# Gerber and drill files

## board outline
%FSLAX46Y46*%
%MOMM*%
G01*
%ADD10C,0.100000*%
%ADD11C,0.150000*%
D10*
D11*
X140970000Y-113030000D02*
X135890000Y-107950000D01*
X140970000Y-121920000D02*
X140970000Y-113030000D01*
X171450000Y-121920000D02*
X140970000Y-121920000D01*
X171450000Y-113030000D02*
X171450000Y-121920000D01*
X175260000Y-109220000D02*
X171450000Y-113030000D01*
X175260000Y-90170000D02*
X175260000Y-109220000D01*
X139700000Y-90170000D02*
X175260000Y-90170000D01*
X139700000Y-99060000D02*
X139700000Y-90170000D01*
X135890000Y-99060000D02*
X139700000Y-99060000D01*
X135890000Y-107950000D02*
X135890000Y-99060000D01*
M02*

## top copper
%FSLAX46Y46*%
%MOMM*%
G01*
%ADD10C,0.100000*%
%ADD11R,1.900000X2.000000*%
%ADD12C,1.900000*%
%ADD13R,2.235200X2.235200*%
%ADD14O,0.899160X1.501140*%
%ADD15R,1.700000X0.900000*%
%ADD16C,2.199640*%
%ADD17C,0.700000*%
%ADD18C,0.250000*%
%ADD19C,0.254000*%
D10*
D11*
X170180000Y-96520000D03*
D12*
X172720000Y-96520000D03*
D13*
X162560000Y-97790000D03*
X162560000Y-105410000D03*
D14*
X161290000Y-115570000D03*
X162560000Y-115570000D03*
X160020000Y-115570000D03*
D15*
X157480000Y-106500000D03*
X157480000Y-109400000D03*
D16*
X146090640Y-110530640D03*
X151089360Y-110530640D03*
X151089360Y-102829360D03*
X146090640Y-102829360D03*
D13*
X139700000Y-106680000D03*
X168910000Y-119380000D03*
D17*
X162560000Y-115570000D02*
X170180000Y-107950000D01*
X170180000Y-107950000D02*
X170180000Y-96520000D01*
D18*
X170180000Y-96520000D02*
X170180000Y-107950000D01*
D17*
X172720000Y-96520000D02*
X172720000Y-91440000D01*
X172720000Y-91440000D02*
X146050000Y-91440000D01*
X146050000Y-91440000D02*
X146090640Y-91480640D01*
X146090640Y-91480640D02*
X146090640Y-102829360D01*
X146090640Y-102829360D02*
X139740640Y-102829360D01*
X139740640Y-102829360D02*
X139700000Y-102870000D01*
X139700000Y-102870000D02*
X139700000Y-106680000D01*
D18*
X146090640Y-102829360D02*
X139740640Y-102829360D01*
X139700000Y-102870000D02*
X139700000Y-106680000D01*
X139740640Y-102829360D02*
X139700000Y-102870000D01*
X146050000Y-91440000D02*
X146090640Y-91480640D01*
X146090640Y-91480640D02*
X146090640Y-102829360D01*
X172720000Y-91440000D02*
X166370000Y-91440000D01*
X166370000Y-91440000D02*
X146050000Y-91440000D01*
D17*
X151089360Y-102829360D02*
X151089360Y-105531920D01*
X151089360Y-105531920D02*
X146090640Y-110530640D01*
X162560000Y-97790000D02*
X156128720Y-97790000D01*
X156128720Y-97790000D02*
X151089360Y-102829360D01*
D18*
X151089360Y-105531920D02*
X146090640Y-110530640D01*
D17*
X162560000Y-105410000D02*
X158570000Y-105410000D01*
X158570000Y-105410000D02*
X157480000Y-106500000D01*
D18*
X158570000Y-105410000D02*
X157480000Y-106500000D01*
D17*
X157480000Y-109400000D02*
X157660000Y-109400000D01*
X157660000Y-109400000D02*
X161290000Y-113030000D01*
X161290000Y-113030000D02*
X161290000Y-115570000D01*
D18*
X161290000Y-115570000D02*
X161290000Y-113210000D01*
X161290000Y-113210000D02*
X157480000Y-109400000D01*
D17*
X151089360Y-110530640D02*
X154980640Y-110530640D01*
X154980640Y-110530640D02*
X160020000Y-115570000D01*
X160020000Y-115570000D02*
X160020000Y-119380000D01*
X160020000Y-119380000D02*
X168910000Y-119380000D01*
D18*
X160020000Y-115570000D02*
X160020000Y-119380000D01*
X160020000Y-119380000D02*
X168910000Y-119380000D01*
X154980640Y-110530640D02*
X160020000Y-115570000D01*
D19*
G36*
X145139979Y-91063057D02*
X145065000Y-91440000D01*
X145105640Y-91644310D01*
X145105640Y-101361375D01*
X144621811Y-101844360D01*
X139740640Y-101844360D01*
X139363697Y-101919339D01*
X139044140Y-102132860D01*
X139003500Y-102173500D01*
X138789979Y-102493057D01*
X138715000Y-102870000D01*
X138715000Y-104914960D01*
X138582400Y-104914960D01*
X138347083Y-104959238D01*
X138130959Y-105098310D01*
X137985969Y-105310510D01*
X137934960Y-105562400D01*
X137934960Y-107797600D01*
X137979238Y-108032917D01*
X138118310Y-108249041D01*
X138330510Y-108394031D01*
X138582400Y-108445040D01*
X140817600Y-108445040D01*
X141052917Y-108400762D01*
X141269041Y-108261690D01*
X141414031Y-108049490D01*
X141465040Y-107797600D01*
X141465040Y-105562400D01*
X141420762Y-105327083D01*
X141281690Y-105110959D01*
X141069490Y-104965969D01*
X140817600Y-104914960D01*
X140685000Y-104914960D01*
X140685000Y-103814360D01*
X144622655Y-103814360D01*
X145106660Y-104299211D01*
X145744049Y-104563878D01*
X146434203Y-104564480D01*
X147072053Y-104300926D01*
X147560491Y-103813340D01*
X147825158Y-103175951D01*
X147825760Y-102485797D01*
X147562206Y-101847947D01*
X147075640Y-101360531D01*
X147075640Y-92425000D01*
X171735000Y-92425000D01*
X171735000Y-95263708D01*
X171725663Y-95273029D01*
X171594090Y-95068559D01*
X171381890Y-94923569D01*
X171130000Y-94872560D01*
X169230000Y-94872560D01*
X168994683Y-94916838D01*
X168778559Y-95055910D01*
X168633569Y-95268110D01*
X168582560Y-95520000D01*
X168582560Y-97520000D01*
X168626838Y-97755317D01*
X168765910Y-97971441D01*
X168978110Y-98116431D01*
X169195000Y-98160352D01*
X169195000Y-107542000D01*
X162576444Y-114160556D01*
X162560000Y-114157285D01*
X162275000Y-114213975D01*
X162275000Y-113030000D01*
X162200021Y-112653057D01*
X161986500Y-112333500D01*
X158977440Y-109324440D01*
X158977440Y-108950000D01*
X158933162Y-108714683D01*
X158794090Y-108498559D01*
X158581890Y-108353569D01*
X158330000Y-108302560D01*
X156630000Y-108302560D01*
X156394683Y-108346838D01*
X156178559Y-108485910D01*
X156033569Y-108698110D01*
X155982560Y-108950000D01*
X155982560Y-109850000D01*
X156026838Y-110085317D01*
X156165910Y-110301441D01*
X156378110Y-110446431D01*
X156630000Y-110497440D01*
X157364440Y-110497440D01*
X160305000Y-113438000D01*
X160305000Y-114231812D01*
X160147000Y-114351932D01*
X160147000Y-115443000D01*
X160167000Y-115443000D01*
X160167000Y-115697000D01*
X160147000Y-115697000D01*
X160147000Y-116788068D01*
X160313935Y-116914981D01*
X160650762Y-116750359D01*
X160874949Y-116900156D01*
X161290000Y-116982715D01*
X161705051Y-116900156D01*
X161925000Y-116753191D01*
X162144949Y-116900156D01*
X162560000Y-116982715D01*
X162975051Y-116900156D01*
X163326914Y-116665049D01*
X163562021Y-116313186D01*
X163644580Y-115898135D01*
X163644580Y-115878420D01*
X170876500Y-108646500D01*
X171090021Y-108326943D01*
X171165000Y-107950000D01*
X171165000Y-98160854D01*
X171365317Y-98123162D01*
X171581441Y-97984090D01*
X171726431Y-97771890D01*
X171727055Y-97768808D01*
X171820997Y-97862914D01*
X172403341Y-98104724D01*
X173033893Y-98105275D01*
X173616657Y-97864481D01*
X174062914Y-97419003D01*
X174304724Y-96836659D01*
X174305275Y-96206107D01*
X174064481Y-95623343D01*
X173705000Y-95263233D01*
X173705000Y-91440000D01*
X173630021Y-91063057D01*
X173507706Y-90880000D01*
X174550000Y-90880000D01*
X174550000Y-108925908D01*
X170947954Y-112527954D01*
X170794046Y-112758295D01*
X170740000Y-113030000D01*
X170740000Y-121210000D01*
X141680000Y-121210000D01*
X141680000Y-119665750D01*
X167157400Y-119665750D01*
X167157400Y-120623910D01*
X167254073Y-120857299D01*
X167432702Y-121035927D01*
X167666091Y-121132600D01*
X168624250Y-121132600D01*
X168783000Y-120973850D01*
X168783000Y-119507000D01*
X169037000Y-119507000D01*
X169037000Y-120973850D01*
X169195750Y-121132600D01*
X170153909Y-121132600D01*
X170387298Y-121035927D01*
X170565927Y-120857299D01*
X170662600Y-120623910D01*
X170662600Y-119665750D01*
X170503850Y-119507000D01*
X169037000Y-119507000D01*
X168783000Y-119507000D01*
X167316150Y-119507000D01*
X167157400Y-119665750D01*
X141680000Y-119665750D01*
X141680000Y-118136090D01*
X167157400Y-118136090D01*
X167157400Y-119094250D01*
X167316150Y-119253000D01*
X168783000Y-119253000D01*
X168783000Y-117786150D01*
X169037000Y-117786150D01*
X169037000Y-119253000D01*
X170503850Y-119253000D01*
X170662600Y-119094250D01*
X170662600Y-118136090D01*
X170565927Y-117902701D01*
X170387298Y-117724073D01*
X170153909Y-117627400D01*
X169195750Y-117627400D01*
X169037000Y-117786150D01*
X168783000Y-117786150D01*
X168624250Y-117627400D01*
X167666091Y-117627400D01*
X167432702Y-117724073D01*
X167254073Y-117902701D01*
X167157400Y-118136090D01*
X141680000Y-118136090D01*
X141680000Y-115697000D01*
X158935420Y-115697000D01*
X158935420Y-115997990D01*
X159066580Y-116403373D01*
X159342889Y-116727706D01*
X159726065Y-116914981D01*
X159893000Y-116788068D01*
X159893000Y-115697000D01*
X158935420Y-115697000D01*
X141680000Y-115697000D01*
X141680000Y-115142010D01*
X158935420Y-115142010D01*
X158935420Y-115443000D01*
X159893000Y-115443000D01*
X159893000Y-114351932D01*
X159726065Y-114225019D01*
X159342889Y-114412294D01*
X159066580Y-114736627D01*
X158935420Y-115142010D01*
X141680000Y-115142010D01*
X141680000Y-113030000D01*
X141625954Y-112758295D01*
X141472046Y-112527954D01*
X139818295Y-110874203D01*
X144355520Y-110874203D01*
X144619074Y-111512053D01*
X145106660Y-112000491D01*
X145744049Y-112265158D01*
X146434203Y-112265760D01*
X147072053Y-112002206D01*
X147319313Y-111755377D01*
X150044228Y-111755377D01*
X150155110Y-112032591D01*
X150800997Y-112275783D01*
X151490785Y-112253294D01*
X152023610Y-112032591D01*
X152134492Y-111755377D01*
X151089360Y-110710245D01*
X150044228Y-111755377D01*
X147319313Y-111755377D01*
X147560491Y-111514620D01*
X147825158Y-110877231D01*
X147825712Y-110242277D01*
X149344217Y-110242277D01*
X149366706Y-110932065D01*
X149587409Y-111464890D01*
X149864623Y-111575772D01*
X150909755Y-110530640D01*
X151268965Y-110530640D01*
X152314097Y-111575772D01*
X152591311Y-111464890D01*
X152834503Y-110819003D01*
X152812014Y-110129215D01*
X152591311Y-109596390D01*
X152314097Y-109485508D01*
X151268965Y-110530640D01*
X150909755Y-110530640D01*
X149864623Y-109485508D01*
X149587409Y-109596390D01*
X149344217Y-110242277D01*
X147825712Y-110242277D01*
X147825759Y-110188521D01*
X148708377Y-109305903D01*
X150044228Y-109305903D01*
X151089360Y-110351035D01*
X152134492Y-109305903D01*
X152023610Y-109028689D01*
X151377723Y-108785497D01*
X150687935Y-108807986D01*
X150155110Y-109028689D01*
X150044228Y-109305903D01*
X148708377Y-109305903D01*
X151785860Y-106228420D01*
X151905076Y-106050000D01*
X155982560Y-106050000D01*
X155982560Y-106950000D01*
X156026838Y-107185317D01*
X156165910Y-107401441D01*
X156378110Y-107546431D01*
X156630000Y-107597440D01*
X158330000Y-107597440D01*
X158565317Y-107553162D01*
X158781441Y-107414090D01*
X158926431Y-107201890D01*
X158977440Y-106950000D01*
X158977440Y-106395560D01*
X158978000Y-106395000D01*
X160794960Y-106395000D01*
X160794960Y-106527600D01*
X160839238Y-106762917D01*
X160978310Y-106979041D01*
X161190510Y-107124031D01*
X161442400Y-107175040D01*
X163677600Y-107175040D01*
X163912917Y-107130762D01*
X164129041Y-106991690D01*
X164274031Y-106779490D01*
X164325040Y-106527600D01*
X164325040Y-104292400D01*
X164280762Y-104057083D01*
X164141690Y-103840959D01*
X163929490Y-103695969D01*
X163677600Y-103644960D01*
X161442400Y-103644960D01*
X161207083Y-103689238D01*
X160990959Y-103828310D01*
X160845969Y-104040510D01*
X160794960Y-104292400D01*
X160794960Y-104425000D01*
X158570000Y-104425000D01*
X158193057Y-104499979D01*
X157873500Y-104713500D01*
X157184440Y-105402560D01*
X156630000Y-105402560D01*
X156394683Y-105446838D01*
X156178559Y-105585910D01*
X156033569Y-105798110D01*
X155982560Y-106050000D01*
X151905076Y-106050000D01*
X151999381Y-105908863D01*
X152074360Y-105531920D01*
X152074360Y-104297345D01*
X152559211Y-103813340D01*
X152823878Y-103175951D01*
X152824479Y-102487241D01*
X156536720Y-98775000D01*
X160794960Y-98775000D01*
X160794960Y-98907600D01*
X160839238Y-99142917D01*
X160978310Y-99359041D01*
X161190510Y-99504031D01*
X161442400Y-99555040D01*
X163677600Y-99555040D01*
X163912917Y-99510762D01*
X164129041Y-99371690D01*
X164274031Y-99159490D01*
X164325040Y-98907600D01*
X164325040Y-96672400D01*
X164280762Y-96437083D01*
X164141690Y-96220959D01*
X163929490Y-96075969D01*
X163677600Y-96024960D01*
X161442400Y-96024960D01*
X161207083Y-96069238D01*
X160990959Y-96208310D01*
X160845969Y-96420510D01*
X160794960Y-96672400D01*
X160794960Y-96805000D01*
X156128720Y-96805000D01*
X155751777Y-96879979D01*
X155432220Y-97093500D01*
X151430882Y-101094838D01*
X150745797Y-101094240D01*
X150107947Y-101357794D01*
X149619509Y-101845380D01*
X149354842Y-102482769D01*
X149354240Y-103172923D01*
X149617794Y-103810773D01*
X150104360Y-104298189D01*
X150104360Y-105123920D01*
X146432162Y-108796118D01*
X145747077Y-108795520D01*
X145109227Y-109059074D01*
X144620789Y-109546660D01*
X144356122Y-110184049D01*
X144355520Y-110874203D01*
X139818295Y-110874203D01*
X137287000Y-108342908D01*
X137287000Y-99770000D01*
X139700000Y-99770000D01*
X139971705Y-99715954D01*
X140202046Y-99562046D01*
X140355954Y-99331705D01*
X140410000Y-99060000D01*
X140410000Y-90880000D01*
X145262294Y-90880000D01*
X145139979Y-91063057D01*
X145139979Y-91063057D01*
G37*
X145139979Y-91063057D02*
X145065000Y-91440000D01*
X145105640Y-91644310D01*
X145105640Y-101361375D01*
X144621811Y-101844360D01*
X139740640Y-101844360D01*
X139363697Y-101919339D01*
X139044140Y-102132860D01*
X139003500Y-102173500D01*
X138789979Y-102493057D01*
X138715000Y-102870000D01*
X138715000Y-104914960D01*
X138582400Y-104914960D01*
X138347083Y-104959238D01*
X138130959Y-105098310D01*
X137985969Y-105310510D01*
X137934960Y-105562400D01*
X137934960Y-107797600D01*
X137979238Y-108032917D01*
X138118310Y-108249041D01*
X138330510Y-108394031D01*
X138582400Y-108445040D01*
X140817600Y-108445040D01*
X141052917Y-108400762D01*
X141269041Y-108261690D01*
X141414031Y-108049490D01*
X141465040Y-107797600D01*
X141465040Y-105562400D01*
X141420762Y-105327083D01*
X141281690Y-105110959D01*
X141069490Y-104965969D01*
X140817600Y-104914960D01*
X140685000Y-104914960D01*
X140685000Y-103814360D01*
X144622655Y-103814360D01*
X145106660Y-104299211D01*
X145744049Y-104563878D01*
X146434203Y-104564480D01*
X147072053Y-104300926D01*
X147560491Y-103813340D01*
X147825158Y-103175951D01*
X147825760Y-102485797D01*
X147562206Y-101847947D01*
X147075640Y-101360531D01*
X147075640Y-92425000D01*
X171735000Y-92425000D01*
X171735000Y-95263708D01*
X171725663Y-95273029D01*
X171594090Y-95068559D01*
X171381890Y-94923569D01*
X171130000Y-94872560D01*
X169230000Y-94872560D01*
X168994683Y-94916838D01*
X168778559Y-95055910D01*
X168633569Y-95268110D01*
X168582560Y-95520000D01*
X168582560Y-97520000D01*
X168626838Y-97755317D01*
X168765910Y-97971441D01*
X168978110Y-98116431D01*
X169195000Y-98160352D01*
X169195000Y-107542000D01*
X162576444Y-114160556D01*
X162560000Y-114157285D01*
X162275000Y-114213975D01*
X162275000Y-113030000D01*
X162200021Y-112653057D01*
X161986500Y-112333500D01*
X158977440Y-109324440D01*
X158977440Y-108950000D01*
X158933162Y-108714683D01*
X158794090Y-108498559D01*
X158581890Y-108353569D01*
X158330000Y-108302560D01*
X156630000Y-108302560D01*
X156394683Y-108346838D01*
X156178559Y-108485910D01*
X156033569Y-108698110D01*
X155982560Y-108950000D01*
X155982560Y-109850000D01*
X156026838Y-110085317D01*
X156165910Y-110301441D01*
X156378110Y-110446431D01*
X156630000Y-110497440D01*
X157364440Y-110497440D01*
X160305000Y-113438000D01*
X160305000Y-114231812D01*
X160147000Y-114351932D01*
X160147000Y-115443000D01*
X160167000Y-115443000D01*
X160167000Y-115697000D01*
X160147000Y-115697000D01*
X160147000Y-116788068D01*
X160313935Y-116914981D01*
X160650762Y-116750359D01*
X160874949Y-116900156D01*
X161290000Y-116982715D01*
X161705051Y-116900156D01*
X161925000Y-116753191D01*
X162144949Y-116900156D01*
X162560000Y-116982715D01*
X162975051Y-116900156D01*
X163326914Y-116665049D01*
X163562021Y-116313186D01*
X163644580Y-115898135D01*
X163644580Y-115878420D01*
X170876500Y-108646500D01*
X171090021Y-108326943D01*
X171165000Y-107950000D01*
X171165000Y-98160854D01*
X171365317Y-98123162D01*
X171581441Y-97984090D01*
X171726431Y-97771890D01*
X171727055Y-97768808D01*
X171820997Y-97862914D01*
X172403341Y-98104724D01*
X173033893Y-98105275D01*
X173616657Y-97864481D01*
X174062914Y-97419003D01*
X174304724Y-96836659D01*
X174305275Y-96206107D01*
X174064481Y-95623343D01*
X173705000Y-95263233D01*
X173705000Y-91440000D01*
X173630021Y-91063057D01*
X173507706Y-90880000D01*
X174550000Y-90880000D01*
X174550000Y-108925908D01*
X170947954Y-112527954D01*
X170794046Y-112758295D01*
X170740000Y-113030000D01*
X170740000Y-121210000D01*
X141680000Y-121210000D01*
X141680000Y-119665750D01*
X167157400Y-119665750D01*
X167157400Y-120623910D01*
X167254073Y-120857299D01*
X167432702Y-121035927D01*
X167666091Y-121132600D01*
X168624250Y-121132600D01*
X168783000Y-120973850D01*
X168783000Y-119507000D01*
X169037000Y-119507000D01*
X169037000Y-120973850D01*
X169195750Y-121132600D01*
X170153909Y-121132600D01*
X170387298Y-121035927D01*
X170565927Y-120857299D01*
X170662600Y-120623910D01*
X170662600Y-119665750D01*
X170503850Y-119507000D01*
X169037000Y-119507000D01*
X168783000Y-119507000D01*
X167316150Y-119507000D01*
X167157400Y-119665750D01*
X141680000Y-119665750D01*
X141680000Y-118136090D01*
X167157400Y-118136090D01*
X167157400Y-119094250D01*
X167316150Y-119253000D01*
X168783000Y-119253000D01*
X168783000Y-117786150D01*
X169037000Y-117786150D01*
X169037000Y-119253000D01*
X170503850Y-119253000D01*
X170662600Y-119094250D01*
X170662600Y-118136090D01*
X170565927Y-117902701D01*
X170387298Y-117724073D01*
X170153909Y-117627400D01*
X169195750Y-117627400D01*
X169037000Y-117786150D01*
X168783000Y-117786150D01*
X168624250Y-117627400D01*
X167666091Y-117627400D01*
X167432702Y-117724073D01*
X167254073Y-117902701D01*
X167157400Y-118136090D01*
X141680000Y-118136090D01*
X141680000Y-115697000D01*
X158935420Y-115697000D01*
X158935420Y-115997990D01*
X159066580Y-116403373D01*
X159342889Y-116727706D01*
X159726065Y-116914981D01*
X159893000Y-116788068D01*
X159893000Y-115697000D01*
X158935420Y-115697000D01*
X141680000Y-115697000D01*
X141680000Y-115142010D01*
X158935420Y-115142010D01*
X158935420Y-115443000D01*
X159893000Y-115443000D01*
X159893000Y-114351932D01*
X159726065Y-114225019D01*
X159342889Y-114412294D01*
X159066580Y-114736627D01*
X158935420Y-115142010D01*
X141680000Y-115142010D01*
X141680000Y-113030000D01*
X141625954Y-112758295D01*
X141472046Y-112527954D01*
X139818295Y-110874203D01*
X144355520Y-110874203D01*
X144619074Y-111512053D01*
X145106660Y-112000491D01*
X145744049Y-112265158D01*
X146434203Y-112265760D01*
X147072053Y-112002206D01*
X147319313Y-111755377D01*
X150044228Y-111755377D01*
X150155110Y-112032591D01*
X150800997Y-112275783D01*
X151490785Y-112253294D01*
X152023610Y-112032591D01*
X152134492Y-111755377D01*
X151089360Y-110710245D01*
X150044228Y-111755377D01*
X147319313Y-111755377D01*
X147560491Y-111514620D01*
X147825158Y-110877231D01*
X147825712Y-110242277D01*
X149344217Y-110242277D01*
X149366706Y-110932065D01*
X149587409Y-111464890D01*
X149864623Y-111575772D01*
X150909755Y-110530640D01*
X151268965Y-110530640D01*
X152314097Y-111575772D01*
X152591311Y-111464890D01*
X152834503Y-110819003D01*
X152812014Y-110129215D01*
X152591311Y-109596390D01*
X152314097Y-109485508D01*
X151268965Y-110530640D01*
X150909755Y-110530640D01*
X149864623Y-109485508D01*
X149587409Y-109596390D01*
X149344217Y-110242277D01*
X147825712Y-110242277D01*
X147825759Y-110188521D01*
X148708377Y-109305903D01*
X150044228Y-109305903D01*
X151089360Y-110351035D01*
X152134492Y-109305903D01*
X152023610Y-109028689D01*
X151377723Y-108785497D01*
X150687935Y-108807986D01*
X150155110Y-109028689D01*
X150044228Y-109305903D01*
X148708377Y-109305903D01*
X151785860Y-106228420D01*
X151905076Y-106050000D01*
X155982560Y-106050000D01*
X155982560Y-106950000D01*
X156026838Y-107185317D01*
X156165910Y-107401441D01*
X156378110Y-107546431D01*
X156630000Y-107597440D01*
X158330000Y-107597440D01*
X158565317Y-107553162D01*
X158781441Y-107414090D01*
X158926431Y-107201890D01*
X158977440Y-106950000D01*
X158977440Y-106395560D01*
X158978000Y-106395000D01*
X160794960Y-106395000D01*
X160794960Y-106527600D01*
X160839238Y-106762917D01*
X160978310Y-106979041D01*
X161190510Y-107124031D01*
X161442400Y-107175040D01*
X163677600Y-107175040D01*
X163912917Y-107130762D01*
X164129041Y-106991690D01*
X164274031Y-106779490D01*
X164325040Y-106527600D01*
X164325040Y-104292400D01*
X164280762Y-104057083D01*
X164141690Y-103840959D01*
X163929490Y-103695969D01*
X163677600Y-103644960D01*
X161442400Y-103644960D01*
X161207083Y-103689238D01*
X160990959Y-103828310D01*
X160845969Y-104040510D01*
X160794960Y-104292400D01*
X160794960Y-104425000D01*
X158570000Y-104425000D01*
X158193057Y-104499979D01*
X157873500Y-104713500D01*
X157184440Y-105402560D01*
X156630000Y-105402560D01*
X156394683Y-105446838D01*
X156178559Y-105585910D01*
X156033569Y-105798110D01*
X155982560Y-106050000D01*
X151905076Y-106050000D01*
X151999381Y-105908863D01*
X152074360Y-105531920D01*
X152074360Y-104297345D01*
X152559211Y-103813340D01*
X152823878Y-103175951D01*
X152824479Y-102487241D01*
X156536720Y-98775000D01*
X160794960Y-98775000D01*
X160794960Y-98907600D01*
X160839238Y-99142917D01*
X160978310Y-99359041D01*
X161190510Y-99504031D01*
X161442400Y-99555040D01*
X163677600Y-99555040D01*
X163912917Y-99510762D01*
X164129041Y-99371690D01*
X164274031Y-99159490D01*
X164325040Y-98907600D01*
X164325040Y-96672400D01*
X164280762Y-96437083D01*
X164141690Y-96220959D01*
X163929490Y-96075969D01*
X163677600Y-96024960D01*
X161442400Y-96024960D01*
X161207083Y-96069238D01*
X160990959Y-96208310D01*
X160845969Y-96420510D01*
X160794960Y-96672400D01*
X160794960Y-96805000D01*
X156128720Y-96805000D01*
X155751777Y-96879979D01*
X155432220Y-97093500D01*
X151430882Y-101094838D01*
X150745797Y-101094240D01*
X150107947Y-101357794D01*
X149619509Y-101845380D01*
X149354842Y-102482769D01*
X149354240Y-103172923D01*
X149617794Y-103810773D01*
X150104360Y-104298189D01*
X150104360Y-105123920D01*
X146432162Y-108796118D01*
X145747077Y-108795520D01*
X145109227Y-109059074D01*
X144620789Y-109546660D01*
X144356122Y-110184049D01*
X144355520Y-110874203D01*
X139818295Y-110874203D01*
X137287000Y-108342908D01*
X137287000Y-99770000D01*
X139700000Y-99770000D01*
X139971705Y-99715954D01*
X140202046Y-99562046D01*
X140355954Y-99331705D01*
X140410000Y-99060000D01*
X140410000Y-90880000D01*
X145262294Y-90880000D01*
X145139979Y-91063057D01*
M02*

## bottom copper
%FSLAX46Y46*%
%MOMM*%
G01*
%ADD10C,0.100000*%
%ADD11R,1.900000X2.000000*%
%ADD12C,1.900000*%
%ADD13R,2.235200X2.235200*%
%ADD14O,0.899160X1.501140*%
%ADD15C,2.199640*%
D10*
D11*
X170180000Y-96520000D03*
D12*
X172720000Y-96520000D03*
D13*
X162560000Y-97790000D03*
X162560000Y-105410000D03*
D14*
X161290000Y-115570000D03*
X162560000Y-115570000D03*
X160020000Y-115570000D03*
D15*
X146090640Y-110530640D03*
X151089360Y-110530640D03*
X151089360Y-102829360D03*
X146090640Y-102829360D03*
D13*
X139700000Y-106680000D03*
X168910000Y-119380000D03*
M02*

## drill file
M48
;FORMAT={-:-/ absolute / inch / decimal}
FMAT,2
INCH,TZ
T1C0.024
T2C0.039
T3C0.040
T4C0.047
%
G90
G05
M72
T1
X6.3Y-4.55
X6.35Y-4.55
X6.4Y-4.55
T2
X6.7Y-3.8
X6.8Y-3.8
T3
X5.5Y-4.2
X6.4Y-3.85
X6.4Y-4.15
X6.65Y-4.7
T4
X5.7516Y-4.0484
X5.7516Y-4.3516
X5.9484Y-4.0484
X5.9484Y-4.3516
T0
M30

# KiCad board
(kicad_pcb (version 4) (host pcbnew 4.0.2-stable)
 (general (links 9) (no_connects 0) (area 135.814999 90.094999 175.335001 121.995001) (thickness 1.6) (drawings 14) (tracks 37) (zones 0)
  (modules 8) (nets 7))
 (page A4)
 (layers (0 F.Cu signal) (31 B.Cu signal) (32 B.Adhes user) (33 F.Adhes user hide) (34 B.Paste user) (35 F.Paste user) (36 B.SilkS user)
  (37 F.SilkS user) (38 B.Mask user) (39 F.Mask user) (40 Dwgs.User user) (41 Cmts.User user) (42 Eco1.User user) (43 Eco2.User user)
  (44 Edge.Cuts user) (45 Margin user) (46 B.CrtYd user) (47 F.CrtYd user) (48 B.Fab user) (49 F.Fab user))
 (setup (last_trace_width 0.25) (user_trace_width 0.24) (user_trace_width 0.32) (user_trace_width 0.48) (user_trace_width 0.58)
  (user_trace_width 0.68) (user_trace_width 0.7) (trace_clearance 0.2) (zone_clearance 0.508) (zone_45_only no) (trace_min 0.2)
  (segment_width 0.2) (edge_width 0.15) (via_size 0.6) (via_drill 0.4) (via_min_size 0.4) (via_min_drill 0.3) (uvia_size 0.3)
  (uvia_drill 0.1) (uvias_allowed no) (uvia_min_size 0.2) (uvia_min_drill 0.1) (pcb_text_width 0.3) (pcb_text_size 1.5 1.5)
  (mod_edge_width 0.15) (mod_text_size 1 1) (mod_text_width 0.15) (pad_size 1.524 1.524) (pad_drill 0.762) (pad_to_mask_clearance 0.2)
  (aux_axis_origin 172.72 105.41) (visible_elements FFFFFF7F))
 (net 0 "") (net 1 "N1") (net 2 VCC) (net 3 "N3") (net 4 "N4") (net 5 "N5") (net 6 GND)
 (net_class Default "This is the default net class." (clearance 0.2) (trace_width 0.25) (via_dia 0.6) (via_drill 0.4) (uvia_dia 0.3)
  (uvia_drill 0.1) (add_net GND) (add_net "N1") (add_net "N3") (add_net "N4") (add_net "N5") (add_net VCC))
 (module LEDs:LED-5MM (layer F.Cu) (at 170.18 96.52)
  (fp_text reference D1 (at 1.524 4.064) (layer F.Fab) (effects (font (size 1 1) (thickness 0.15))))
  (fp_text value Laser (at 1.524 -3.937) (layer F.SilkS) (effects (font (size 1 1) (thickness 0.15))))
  (pad 1 thru_hole rect (at 0 0 90) (size 2 1.9) (drill 1.00076) (layers *.Cu *.Mask F.SilkS) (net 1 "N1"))
  (pad 2 thru_hole circle (at 2.54 0) (size 1.9 1.9) (drill 1.00076) (layers *.Cu *.Mask F.SilkS) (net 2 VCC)))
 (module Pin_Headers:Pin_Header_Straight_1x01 (layer F.Cu) (at 162.56 97.79)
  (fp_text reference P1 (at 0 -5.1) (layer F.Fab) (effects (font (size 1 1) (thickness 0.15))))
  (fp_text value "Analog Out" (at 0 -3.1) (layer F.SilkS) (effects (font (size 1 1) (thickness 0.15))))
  (pad 1 thru_hole rect (at 0 0) (size 2.2352 2.2352) (drill 1.016) (layers *.Cu *.Mask F.SilkS) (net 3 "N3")))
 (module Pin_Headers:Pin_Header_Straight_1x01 (layer F.Cu) (at 162.56 105.41)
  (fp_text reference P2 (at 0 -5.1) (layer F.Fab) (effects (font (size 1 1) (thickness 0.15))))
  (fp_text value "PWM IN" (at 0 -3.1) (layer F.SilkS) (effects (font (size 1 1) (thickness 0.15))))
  (pad 1 thru_hole rect (at 0 0) (size 2.2352 2.2352) (drill 1.016) (layers *.Cu *.Mask F.SilkS) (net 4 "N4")))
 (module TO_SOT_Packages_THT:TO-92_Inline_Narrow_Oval (layer F.Cu) (at 160.02 115.57)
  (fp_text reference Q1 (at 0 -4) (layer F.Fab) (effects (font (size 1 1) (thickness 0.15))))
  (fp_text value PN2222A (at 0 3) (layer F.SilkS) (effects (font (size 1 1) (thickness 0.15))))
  (pad 2 thru_hole oval (at 1.27 0 180) (size 0.89916 1.50114) (drill 0.6) (layers *.Cu *.Mask F.SilkS) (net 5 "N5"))
  (pad 3 thru_hole oval (at 2.54 0 180) (size 0.89916 1.50114) (drill 0.6) (layers *.Cu *.Mask F.SilkS) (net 1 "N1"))
  (pad 1 thru_hole oval (at 0 0 180) (size 0.89916 1.50114) (drill 0.6) (layers *.Cu *.Mask F.SilkS) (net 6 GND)))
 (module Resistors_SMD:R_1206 (layer F.Cu) (at 157.48 107.95 270)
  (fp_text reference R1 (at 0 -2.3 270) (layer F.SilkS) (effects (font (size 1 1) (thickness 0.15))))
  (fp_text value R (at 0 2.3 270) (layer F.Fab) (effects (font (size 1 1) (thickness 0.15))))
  (pad 1 smd rect (at -1.45 0 270) (size 0.9 1.7) (layers F.Cu F.Paste F.Mask) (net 4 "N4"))
  (pad 2 smd rect (at 1.45 0 270) (size 0.9 1.7) (layers F.Cu F.Paste F.Mask) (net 5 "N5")))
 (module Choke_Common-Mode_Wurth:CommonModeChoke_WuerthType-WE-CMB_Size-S (layer F.Cu) (at 148.59 106.68)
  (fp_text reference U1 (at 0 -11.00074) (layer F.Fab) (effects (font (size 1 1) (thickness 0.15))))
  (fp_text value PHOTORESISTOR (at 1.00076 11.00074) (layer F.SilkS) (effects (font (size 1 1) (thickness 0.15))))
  (pad 4 thru_hole circle (at -2.49936 3.85064) (size 2.19964 2.19964) (drill 1.19888) (layers *.Cu *.Mask F.SilkS) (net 3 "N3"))
  (pad 3 thru_hole circle (at 2.49936 3.85064) (size 2.19964 2.19964) (drill 1.19888) (layers *.Cu *.Mask F.SilkS) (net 6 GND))
  (pad 2 thru_hole circle (at 2.49936 -3.85064) (size 2.19964 2.19964) (drill 1.19888) (layers *.Cu *.Mask F.SilkS) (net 3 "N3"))
  (pad 1 thru_hole circle (at -2.49936 -3.85064) (size 2.19964 2.19964) (drill 1.19888) (layers *.Cu *.Mask F.SilkS) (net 2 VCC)))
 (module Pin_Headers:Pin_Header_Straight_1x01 (layer F.Cu) (at 139.7 106.68)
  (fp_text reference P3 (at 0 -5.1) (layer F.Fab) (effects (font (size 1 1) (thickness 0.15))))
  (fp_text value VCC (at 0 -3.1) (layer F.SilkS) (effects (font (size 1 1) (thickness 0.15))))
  (pad 1 thru_hole rect (at 0 0) (size 2.2352 2.2352) (drill 1.016) (layers *.Cu *.Mask F.SilkS) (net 2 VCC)))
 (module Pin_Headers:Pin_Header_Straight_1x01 (layer F.Cu) (at 168.91 119.38)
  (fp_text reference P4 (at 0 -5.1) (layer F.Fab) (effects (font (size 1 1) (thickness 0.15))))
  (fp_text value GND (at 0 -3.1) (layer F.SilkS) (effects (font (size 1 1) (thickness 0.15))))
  (pad 1 thru_hole rect (at 0 0) (size 2.2352 2.2352) (drill 1.016) (layers *.Cu *.Mask F.SilkS) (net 6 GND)))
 (gr_circle (center 172.72 105.41) (end 172.72 104.14) (layer Edge.Cuts) (width 0.15))
 (gr_line (start 140.97 113.03) (end 135.89 107.95) (angle 90) (layer Edge.Cuts) (width 0.15))
 (gr_line (start 140.97 121.92) (end 140.97 113.03) (angle 90) (layer Edge.Cuts) (width 0.15))
 (gr_line (start 171.45 121.92) (end 140.97 121.92) (angle 90) (layer Edge.Cuts) (width 0.15))
 (gr_line (start 171.45 113.03) (end 171.45 121.92) (angle 90) (layer Edge.Cuts) (width 0.15))
 (gr_line (start 175.26 109.22) (end 171.45 113.03) (angle 90) (layer Edge.Cuts) (width 0.15))
 (gr_line (start 175.26 90.17) (end 175.26 109.22) (angle 90) (layer Edge.Cuts) (width 0.15))
 (gr_line (start 139.7 90.17) (end 175.26 90.17) (angle 90) (layer Edge.Cuts) (width 0.15))
 (gr_line (start 139.7 99.06) (end 139.7 90.17) (angle 90) (layer Edge.Cuts) (width 0.15))
 (gr_line (start 135.89 99.06) (end 139.7 99.06) (angle 90) (layer Edge.Cuts) (width 0.15))
 (gr_line (start 135.89 107.95) (end 135.89 99.06) (angle 90) (layer Edge.Cuts) (width 0.15))
 (segment (start 162.56 115.57) (end 170.18 107.95) (width 0.7) (layer F.Cu) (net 1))
 (segment (start 170.18 107.95) (end 170.18 96.52) (width 0.7) (layer F.Cu) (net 1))
 (segment (start 170.18 96.52) (end 170.18 107.95) (width 0.25) (layer F.Cu) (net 1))
 (segment (start 172.72 96.52) (end 172.72 91.44) (width 0.7) (layer F.Cu) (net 2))
 (segment (start 172.72 91.44) (end 146.05 91.44) (width 0.7) (layer F.Cu) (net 2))
 (segment (start 146.05 91.44) (end 146.09064 91.48064) (width 0.7) (layer F.Cu) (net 2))
 (segment (start 146.09064 91.48064) (end 146.09064 102.82936) (width 0.7) (layer F.Cu) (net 2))
 (segment (start 146.09064 102.82936) (end 139.74064 102.82936) (width 0.7) (layer F.Cu) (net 2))
 (segment (start 139.74064 102.82936) (end 139.7 102.87) (width 0.7) (layer F.Cu) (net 2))
 (segment (start 139.7 102.87) (end 139.7 106.68) (width 0.7) (layer F.Cu) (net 2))
 (segment (start 146.09064 102.82936) (end 139.74064 102.82936) (width 0.25) (layer F.Cu) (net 2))
 (segment (start 139.7 102.87) (end 139.7 106.68) (width 0.25) (layer F.Cu) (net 2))
 (segment (start 139.74064 102.82936) (end 139.7 102.87) (width 0.25) (layer F.Cu) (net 2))
 (segment (start 146.05 91.44) (end 146.09064 91.48064) (width 0.25) (layer F.Cu) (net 2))
 (segment (start 146.09064 91.48064) (end 146.09064 102.82936) (width 0.25) (layer F.Cu) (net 2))
 (segment (start 172.72 91.44) (end 166.37 91.44) (width 0.25) (layer F.Cu) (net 2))
 (segment (start 166.37 91.44) (end 146.05 91.44) (width 0.25) (layer F.Cu) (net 2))
 (segment (start 151.08936 102.82936) (end 151.08936 105.53192) (width 0.7) (layer F.Cu) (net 3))
 (segment (start 151.08936 105.53192) (end 146.09064 110.53064) (width 0.7) (layer F.Cu) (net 3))
 (segment (start 162.56 97.79) (end 156.12872 97.79) (width 0.7) (layer F.Cu) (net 3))
 (segment (start 156.12872 97.79) (end 151.08936 102.82936) (width 0.7) (layer F.Cu) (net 3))
 (segment (start 151.08936 105.53192) (end 146.09064 110.53064) (width 0.25) (layer F.Cu) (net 3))
 (segment (start 162.56 105.41) (end 158.57 105.41) (width 0.7) (layer F.Cu) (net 4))
 (segment (start 158.57 105.41) (end 157.48 106.5) (width 0.7) (layer F.Cu) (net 4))
 (segment (start 158.57 105.41) (end 157.48 106.5) (width 0.25) (layer F.Cu) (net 4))
 (segment (start 157.48 109.4) (end 157.66 109.4) (width 0.7) (layer F.Cu) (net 5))
 (segment (start 157.66 109.4) (end 161.29 113.03) (width 0.7) (layer F.Cu) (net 5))
 (segment (start 161.29 113.03) (end 161.29 115.57) (width 0.7) (layer F.Cu) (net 5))
 (segment (start 161.29 115.57) (end 161.29 113.21) (width 0.25) (layer F.Cu) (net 5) (status 10))
 (segment (start 161.29 113.21) (end 157.48 109.4) (width 0.25) (layer F.Cu) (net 5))
 (segment (start 151.08936 110.53064) (end 154.98064 110.53064) (width 0.7) (layer F.Cu) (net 6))
 (segment (start 154.98064 110.53064) (end 160.02 115.57) (width 0.7) (layer F.Cu) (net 6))
 (segment (start 160.02 115.57) (end 160.02 119.38) (width 0.7) (layer F.Cu) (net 6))
 (segment (start 160.02 119.38) (end 168.91 119.38) (width 0.7) (layer F.Cu) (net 6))
 (segment (start 160.02 115.57) (end 160.02 119.38) (width 0.25) (layer F.Cu) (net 6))
 (segment (start 160.02 119.38) (end 168.91 119.38) (width 0.25) (layer F.Cu) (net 6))
 (segment (start 154.98064 110.53064) (end 160.02 115.57) (width 0.25) (layer F.Cu) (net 6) (status 20))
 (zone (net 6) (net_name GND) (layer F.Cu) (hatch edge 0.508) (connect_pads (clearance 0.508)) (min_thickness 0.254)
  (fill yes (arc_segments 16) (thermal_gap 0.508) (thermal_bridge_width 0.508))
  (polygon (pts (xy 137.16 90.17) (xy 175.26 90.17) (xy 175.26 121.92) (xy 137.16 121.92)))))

